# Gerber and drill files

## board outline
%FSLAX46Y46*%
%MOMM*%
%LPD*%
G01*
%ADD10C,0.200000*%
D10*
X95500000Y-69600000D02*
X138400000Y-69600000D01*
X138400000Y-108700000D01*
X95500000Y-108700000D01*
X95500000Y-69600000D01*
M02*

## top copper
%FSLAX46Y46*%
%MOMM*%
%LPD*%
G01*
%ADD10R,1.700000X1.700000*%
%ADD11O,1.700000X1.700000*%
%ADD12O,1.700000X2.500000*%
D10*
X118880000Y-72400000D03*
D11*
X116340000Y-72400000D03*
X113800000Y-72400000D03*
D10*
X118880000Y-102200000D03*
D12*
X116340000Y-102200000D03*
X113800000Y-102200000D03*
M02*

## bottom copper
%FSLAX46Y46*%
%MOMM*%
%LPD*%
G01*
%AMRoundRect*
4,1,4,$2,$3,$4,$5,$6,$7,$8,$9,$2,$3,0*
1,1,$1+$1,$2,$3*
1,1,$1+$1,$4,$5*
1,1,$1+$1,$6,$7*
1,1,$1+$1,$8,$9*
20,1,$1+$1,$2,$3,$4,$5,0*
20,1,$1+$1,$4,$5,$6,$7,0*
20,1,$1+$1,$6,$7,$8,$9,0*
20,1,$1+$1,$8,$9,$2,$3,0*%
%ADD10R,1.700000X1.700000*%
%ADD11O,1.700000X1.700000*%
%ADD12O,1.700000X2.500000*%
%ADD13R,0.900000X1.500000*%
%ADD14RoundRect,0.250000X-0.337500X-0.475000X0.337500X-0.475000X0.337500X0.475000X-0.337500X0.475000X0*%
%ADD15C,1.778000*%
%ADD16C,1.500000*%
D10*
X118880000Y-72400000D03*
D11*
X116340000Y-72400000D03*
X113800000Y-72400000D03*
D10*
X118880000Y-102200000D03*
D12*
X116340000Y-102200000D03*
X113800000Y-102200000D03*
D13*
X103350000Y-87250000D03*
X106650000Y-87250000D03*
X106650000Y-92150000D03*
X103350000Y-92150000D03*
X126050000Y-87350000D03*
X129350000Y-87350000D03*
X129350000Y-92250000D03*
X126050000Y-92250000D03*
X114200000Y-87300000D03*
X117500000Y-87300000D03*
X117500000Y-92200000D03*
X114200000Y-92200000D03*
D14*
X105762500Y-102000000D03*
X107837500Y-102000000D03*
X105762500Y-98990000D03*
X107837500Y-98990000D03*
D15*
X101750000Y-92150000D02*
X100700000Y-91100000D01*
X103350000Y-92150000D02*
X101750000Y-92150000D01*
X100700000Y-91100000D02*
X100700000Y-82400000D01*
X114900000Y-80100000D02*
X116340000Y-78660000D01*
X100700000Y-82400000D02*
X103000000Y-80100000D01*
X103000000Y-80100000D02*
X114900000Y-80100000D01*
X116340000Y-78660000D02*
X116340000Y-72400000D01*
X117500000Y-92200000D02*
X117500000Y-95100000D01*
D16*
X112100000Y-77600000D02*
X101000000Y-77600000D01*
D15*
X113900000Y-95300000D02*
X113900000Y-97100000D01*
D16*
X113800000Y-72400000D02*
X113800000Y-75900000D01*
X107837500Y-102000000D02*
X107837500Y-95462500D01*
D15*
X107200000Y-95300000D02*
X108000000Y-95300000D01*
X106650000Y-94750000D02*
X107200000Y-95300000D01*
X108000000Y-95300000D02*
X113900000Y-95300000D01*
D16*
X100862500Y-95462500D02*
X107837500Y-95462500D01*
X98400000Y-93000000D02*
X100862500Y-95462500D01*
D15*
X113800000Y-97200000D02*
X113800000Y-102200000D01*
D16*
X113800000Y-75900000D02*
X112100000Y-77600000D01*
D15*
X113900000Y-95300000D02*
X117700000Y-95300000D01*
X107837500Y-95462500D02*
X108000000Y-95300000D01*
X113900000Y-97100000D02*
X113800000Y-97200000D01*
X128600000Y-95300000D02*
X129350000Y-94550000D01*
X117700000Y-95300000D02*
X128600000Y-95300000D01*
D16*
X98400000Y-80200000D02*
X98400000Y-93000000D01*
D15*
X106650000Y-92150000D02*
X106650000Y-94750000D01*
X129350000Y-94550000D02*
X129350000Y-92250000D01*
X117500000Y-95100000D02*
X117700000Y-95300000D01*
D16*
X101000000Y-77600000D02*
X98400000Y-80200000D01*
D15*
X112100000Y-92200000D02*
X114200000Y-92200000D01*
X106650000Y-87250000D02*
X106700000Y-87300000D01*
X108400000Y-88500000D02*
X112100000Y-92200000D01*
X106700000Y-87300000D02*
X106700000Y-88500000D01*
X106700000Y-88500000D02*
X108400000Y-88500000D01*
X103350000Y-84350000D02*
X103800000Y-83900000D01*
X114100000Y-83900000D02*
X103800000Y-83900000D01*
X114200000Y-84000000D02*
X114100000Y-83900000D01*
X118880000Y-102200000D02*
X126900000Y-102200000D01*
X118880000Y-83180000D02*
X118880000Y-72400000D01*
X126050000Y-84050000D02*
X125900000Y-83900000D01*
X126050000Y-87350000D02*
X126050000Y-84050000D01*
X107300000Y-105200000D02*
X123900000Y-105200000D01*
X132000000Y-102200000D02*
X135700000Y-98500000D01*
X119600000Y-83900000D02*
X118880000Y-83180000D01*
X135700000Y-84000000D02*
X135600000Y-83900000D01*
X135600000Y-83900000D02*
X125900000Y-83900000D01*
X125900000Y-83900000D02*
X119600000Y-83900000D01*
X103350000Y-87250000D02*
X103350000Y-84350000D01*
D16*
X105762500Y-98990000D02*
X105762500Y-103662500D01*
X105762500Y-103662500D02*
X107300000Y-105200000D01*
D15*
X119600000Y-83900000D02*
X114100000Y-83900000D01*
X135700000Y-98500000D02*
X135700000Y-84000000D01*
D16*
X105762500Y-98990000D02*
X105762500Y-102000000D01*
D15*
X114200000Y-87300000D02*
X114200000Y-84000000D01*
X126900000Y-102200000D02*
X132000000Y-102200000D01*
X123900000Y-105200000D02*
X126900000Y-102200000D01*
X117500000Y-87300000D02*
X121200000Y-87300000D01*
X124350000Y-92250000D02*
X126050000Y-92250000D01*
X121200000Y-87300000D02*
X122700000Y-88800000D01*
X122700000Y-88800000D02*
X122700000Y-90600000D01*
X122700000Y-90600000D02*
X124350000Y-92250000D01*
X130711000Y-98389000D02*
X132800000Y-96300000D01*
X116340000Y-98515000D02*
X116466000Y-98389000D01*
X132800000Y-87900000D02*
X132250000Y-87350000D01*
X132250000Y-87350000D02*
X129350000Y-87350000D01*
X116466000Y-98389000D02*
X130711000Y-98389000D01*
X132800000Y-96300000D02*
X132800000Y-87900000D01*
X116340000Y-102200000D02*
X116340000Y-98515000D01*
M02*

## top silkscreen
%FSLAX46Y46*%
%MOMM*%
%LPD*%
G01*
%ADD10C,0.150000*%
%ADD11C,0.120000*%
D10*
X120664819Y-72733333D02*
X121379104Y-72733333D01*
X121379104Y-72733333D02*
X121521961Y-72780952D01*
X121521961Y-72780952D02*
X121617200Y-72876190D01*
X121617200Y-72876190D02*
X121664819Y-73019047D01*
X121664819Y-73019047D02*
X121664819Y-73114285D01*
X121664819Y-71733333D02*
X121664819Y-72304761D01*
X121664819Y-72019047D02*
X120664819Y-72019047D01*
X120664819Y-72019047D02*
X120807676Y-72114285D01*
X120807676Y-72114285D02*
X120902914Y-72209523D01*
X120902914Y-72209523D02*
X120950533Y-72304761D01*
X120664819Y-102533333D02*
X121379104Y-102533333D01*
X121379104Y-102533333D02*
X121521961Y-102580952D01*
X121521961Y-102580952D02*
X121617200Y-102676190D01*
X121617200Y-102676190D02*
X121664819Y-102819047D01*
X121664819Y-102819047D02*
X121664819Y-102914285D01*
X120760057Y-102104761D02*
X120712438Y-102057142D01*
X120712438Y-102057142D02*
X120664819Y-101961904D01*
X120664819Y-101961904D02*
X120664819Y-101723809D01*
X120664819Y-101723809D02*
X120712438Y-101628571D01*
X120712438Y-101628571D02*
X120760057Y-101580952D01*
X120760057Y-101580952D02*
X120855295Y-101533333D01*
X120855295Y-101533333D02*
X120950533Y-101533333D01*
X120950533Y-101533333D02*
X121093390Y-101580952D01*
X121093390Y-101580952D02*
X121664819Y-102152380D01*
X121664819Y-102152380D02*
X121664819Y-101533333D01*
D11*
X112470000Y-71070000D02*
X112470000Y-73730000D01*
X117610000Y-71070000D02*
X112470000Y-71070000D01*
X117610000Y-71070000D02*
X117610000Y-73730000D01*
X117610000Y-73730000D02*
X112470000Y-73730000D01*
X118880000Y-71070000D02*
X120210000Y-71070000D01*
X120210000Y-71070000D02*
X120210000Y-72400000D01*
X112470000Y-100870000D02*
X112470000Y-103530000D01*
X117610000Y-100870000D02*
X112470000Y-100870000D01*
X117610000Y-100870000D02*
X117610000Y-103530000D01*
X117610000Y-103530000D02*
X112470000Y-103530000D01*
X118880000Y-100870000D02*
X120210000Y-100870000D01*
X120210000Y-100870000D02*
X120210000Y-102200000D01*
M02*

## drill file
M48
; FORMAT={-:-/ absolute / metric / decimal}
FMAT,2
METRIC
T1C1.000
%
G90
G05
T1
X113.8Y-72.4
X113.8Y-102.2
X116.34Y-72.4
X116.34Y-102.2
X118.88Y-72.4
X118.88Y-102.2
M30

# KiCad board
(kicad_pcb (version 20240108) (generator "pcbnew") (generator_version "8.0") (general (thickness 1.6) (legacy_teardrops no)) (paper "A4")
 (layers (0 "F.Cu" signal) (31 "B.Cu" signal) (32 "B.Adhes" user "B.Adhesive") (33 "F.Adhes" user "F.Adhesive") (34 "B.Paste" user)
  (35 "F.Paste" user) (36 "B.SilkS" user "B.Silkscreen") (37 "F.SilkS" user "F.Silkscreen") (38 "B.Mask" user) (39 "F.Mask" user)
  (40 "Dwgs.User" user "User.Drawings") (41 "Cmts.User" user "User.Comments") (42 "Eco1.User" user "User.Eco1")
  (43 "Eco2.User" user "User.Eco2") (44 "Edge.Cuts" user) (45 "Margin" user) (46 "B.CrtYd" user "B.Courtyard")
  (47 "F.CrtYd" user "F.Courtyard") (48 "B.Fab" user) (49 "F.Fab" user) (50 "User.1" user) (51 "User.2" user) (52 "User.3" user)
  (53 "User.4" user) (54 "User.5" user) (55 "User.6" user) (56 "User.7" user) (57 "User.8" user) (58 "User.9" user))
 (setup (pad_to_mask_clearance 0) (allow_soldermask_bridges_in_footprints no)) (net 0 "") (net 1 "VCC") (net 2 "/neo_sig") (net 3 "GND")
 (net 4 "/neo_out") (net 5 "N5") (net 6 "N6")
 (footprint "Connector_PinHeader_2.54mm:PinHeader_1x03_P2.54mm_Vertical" (layer "F.Cu") (at 118.88 72.4 -90)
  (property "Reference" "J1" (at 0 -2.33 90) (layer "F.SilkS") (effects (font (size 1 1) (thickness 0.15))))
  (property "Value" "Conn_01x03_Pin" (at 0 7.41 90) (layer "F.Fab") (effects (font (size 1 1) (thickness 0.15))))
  (fp_line (start -1.33 6.41) (end 1.33 6.41) (stroke (width 0.12) (type solid)) (layer "F.SilkS"))
  (fp_line (start -1.33 1.27) (end -1.33 6.41) (stroke (width 0.12) (type solid)) (layer "F.SilkS"))
  (fp_line (start -1.33 1.27) (end 1.33 1.27) (stroke (width 0.12) (type solid)) (layer "F.SilkS"))
  (fp_line (start 1.33 1.27) (end 1.33 6.41) (stroke (width 0.12) (type solid)) (layer "F.SilkS"))
  (fp_line (start -1.33 0) (end -1.33 -1.33) (stroke (width 0.12) (type solid)) (layer "F.SilkS"))
  (fp_line (start -1.33 -1.33) (end 0 -1.33) (stroke (width 0.12) (type solid)) (layer "F.SilkS"))
  (pad "1" thru_hole rect (at 0 0 270) (size 1.7 1.7) (drill 1) (layers "*.Cu" "*.Mask") (remove_unused_layers no) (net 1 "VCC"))
  (pad "2" thru_hole oval (at 0 2.54 270) (size 1.7 1.7) (drill 1) (layers "*.Cu" "*.Mask") (remove_unused_layers no) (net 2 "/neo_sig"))
  (pad "3" thru_hole oval (at 0 5.08 270) (size 1.7 1.7) (drill 1) (layers "*.Cu" "*.Mask") (remove_unused_layers no) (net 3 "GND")))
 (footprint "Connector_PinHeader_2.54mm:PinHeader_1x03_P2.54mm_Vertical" (layer "F.Cu") (at 118.88 102.2 -90)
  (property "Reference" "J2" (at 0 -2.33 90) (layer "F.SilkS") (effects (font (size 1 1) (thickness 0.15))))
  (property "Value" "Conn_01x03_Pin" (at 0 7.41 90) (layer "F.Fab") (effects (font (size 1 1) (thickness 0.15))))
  (fp_line (start -1.33 6.41) (end 1.33 6.41) (stroke (width 0.12) (type solid)) (layer "F.SilkS"))
  (fp_line (start -1.33 1.27) (end -1.33 6.41) (stroke (width 0.12) (type solid)) (layer "F.SilkS"))
  (fp_line (start -1.33 1.27) (end 1.33 1.27) (stroke (width 0.12) (type solid)) (layer "F.SilkS"))
  (fp_line (start 1.33 1.27) (end 1.33 6.41) (stroke (width 0.12) (type solid)) (layer "F.SilkS"))
  (fp_line (start -1.33 0) (end -1.33 -1.33) (stroke (width 0.12) (type solid)) (layer "F.SilkS"))
  (fp_line (start -1.33 -1.33) (end 0 -1.33) (stroke (width 0.12) (type solid)) (layer "F.SilkS"))
  (pad "1" thru_hole rect (at 0 0 270) (size 1.7 1.7) (drill 1) (layers "*.Cu" "*.Mask") (remove_unused_layers no) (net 1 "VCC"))
  (pad "2" thru_hole oval (at 0 2.54 270) (size 2.5 1.7) (drill 1) (layers "*.Cu" "*.Mask") (remove_unused_layers no) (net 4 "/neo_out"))
  (pad "3" thru_hole oval (at 0 5.08 270) (size 2.5 1.7) (drill 1) (layers "*.Cu" "*.Mask") (remove_unused_layers no) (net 3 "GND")))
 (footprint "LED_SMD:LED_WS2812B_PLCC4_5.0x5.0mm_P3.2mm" (layer "B.Cu") (at 105 89.7 -90)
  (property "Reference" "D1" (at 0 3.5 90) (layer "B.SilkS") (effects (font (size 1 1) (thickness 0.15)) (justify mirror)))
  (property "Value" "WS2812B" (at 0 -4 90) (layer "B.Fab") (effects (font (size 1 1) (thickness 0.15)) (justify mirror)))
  (pad "1" smd rect (at -2.45 1.65 270) (size 1.5 0.9) (layers "B.Cu" "B.Paste" "B.Mask") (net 1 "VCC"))
  (pad "2" smd rect (at -2.45 -1.65 270) (size 1.5 0.9) (layers "B.Cu" "B.Paste" "B.Mask") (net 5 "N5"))
  (pad "3" smd rect (at 2.45 -1.65 270) (size 1.5 0.9) (layers "B.Cu" "B.Paste" "B.Mask") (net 3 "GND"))
  (pad "4" smd rect (at 2.45 1.65 270) (size 1.5 0.9) (layers "B.Cu" "B.Paste" "B.Mask") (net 2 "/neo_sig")))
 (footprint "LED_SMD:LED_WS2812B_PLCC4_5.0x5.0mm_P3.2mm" (layer "B.Cu") (at 127.7 89.8 -90)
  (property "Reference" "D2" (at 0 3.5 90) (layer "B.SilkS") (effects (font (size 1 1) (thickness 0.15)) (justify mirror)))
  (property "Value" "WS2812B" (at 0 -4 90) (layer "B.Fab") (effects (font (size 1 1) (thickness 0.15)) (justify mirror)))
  (pad "1" smd rect (at -2.45 1.65 270) (size 1.5 0.9) (layers "B.Cu" "B.Paste" "B.Mask") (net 1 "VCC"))
  (pad "2" smd rect (at -2.45 -1.65 270) (size 1.5 0.9) (layers "B.Cu" "B.Paste" "B.Mask") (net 4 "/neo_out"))
  (pad "3" smd rect (at 2.45 -1.65 270) (size 1.5 0.9) (layers "B.Cu" "B.Paste" "B.Mask") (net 3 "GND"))
  (pad "4" smd rect (at 2.45 1.65 270) (size 1.5 0.9) (layers "B.Cu" "B.Paste" "B.Mask") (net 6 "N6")))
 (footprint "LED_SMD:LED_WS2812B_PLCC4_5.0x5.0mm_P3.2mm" (layer "B.Cu") (at 115.85 89.75 -90)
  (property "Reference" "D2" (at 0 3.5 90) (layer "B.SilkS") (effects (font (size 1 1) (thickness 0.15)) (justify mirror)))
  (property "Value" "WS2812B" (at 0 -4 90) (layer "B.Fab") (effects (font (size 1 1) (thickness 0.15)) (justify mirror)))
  (pad "1" smd rect (at -2.45 1.65 270) (size 1.5 0.9) (layers "B.Cu" "B.Paste" "B.Mask") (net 1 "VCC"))
  (pad "2" smd rect (at -2.45 -1.65 270) (size 1.5 0.9) (layers "B.Cu" "B.Paste" "B.Mask") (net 6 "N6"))
  (pad "3" smd rect (at 2.45 -1.65 270) (size 1.5 0.9) (layers "B.Cu" "B.Paste" "B.Mask") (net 3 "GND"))
  (pad "4" smd rect (at 2.45 1.65 270) (size 1.5 0.9) (layers "B.Cu" "B.Paste" "B.Mask") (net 5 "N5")))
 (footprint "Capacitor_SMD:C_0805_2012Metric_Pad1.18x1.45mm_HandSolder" (layer "B.Cu") (at 106.8 102)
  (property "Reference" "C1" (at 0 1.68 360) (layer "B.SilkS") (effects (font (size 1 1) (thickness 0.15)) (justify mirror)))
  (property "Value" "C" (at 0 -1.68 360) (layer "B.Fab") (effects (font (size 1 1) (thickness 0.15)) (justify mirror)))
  (pad "1" smd roundrect (at -1.0375 0) (size 1.175 1.45) (layers "B.Cu" "B.Paste" "B.Mask") (roundrect_rratio 0.212766) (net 1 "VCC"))
  (pad "2" smd roundrect (at 1.0375 0) (size 1.175 1.45) (layers "B.Cu" "B.Paste" "B.Mask") (roundrect_rratio 0.212766) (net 3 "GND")))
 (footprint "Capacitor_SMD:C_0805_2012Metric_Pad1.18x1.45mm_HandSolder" (layer "B.Cu") (at 106.8 98.99)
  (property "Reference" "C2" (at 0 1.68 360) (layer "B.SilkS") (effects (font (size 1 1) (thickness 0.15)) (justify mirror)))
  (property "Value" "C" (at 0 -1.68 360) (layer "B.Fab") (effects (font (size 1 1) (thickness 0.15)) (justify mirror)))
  (pad "1" smd roundrect (at -1.0375 0) (size 1.175 1.45) (layers "B.Cu" "B.Paste" "B.Mask") (roundrect_rratio 0.212766) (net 1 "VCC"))
  (pad "2" smd roundrect (at 1.0375 0) (size 1.175 1.45) (layers "B.Cu" "B.Paste" "B.Mask") (roundrect_rratio 0.212766) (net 3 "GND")))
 (gr_rect (start 95.5 69.6) (end 138.4 108.7) (stroke (width 0.2) (type default)) (fill none) (layer "Edge.Cuts"))
 (segment (start 101.75 92.15) (end 100.7 91.1) (width 1.778) (layer "B.Cu") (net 2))
 (segment (start 103.35 92.15) (end 101.75 92.15) (width 1.778) (layer "B.Cu") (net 2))
 (segment (start 100.7 91.1) (end 100.7 82.4) (width 1.778) (layer "B.Cu") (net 2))
 (segment (start 114.9 80.1) (end 116.34 78.66) (width 1.778) (layer "B.Cu") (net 2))
 (segment (start 100.7 82.4) (end 103 80.1) (width 1.778) (layer "B.Cu") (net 2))
 (segment (start 103 80.1) (end 114.9 80.1) (width 1.778) (layer "B.Cu") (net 2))
 (segment (start 116.34 78.66) (end 116.34 72.4) (width 1.778) (layer "B.Cu") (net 2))
 (segment (start 117.5 92.2) (end 117.5 95.1) (width 1.778) (layer "B.Cu") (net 3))
 (segment (start 112.1 77.6) (end 101 77.6) (width 1.5) (layer "B.Cu") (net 3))
 (segment (start 113.9 95.3) (end 113.9 97.1) (width 1.778) (layer "B.Cu") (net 3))
 (segment (start 113.8 72.4) (end 113.8 75.9) (width 1.5) (layer "B.Cu") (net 3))
 (segment (start 107.8375 102) (end 107.8375 95.4625) (width 1.5) (layer "B.Cu") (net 3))
 (segment (start 107.2 95.3) (end 108 95.3) (width 1.778) (layer "B.Cu") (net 3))
 (segment (start 106.65 94.75) (end 107.2 95.3) (width 1.778) (layer "B.Cu") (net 3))
 (segment (start 108 95.3) (end 113.9 95.3) (width 1.778) (layer "B.Cu") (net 3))
 (segment (start 100.8625 95.4625) (end 107.8375 95.4625) (width 1.5) (layer "B.Cu") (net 3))
 (segment (start 98.4 93) (end 100.8625 95.4625) (width 1.5) (layer "B.Cu") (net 3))
 (segment (start 113.8 97.2) (end 113.8 102.2) (width 1.778) (layer "B.Cu") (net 3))
 (segment (start 113.8 75.9) (end 112.1 77.6) (width 1.5) (layer "B.Cu") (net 3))
 (segment (start 113.9 95.3) (end 117.7 95.3) (width 1.778) (layer "B.Cu") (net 3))
 (segment (start 107.8375 95.4625) (end 108 95.3) (width 1.778) (layer "B.Cu") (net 3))
 (segment (start 113.9 97.1) (end 113.8 97.2) (width 1.778) (layer "B.Cu") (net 3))
 (segment (start 128.6 95.3) (end 129.35 94.55) (width 1.778) (layer "B.Cu") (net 3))
 (segment (start 117.7 95.3) (end 128.6 95.3) (width 1.778) (layer "B.Cu") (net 3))
 (segment (start 98.4 80.2) (end 98.4 93) (width 1.5) (layer "B.Cu") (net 3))
 (segment (start 106.65 92.15) (end 106.65 94.75) (width 1.778) (layer "B.Cu") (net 3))
 (segment (start 129.35 94.55) (end 129.35 92.25) (width 1.778) (layer "B.Cu") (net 3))
 (segment (start 117.5 95.1) (end 117.7 95.3) (width 1.778) (layer "B.Cu") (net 3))
 (segment (start 101 77.6) (end 98.4 80.2) (width 1.5) (layer "B.Cu") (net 3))
 (segment (start 112.1 92.2) (end 114.2 92.2) (width 1.778) (layer "B.Cu") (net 5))
 (segment (start 106.65 87.25) (end 106.7 87.3) (width 1.778) (layer "B.Cu") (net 5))
 (segment (start 108.4 88.5) (end 112.1 92.2) (width 1.778) (layer "B.Cu") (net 5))
 (segment (start 106.7 87.3) (end 106.7 88.5) (width 1.778) (layer "B.Cu") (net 5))
 (segment (start 106.7 88.5) (end 108.4 88.5) (width 1.778) (layer "B.Cu") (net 5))
 (segment (start 103.35 84.35) (end 103.8 83.9) (width 1.778) (layer "B.Cu") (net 1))
 (segment (start 114.1 83.9) (end 103.8 83.9) (width 1.778) (layer "B.Cu") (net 1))
 (segment (start 114.2 84) (end 114.1 83.9) (width 1.778) (layer "B.Cu") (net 1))
 (segment (start 118.88 102.2) (end 126.9 102.2) (width 1.778) (layer "B.Cu") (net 1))
 (segment (start 118.88 83.18) (end 118.88 72.4) (width 1.778) (layer "B.Cu") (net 1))
 (segment (start 126.05 84.05) (end 125.9 83.9) (width 1.778) (layer "B.Cu") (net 1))
 (segment (start 126.05 87.35) (end 126.05 84.05) (width 1.778) (layer "B.Cu") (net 1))
 (segment (start 107.3 105.2) (end 123.9 105.2) (width 1.778) (layer "B.Cu") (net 1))
 (segment (start 132 102.2) (end 135.7 98.5) (width 1.778) (layer "B.Cu") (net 1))
 (segment (start 119.6 83.9) (end 118.88 83.18) (width 1.778) (layer "B.Cu") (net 1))
 (segment (start 135.7 84) (end 135.6 83.9) (width 1.778) (layer "B.Cu") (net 1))
 (segment (start 135.6 83.9) (end 125.9 83.9) (width 1.778) (layer "B.Cu") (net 1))
 (segment (start 125.9 83.9) (end 119.6 83.9) (width 1.778) (layer "B.Cu") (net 1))
 (segment (start 103.35 87.25) (end 103.35 84.35) (width 1.778) (layer "B.Cu") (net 1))
 (segment (start 105.7625 98.99) (end 105.7625 103.6625) (width 1.5) (layer "B.Cu") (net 1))
 (segment (start 105.7625 103.6625) (end 107.3 105.2) (width 1.5) (layer "B.Cu") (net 1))
 (segment (start 119.6 83.9) (end 114.1 83.9) (width 1.778) (layer "B.Cu") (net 1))
 (segment (start 135.7 98.5) (end 135.7 84) (width 1.778) (layer "B.Cu") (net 1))
 (segment (start 105.7625 98.99) (end 105.7625 102) (width 1.5) (layer "B.Cu") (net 1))
 (segment (start 114.2 87.3) (end 114.2 84) (width 1.778) (layer "B.Cu") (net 1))
 (segment (start 126.9 102.2) (end 132 102.2) (width 1.778) (layer "B.Cu") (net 1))
 (segment (start 123.9 105.2) (end 126.9 102.2) (width 1.778) (layer "B.Cu") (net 1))
 (segment (start 117.5 87.3) (end 121.2 87.3) (width 1.778) (layer "B.Cu") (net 6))
 (segment (start 124.35 92.25) (end 126.05 92.25) (width 1.778) (layer "B.Cu") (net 6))
 (segment (start 121.2 87.3) (end 122.7 88.8) (width 1.778) (layer "B.Cu") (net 6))
 (segment (start 122.7 88.8) (end 122.7 90.6) (width 1.778) (layer "B.Cu") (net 6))
 (segment (start 122.7 90.6) (end 124.35 92.25) (width 1.778) (layer "B.Cu") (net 6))
 (segment (start 130.711 98.389) (end 132.8 96.3) (width 1.778) (layer "B.Cu") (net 4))
 (segment (start 116.34 98.515) (end 116.466 98.389) (width 1.778) (layer "B.Cu") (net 4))
 (segment (start 132.8 87.9) (end 132.25 87.35) (width 1.778) (layer "B.Cu") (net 4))
 (segment (start 132.25 87.35) (end 129.35 87.35) (width 1.778) (layer "B.Cu") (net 4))
 (segment (start 116.466 98.389) (end 130.711 98.389) (width 1.778) (layer "B.Cu") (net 4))
 (segment (start 132.8 96.3) (end 132.8 87.9) (width 1.778) (layer "B.Cu") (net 4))
 (segment (start 116.34 102.2) (end 116.34 98.515) (width 1.778) (layer "B.Cu") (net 4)))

